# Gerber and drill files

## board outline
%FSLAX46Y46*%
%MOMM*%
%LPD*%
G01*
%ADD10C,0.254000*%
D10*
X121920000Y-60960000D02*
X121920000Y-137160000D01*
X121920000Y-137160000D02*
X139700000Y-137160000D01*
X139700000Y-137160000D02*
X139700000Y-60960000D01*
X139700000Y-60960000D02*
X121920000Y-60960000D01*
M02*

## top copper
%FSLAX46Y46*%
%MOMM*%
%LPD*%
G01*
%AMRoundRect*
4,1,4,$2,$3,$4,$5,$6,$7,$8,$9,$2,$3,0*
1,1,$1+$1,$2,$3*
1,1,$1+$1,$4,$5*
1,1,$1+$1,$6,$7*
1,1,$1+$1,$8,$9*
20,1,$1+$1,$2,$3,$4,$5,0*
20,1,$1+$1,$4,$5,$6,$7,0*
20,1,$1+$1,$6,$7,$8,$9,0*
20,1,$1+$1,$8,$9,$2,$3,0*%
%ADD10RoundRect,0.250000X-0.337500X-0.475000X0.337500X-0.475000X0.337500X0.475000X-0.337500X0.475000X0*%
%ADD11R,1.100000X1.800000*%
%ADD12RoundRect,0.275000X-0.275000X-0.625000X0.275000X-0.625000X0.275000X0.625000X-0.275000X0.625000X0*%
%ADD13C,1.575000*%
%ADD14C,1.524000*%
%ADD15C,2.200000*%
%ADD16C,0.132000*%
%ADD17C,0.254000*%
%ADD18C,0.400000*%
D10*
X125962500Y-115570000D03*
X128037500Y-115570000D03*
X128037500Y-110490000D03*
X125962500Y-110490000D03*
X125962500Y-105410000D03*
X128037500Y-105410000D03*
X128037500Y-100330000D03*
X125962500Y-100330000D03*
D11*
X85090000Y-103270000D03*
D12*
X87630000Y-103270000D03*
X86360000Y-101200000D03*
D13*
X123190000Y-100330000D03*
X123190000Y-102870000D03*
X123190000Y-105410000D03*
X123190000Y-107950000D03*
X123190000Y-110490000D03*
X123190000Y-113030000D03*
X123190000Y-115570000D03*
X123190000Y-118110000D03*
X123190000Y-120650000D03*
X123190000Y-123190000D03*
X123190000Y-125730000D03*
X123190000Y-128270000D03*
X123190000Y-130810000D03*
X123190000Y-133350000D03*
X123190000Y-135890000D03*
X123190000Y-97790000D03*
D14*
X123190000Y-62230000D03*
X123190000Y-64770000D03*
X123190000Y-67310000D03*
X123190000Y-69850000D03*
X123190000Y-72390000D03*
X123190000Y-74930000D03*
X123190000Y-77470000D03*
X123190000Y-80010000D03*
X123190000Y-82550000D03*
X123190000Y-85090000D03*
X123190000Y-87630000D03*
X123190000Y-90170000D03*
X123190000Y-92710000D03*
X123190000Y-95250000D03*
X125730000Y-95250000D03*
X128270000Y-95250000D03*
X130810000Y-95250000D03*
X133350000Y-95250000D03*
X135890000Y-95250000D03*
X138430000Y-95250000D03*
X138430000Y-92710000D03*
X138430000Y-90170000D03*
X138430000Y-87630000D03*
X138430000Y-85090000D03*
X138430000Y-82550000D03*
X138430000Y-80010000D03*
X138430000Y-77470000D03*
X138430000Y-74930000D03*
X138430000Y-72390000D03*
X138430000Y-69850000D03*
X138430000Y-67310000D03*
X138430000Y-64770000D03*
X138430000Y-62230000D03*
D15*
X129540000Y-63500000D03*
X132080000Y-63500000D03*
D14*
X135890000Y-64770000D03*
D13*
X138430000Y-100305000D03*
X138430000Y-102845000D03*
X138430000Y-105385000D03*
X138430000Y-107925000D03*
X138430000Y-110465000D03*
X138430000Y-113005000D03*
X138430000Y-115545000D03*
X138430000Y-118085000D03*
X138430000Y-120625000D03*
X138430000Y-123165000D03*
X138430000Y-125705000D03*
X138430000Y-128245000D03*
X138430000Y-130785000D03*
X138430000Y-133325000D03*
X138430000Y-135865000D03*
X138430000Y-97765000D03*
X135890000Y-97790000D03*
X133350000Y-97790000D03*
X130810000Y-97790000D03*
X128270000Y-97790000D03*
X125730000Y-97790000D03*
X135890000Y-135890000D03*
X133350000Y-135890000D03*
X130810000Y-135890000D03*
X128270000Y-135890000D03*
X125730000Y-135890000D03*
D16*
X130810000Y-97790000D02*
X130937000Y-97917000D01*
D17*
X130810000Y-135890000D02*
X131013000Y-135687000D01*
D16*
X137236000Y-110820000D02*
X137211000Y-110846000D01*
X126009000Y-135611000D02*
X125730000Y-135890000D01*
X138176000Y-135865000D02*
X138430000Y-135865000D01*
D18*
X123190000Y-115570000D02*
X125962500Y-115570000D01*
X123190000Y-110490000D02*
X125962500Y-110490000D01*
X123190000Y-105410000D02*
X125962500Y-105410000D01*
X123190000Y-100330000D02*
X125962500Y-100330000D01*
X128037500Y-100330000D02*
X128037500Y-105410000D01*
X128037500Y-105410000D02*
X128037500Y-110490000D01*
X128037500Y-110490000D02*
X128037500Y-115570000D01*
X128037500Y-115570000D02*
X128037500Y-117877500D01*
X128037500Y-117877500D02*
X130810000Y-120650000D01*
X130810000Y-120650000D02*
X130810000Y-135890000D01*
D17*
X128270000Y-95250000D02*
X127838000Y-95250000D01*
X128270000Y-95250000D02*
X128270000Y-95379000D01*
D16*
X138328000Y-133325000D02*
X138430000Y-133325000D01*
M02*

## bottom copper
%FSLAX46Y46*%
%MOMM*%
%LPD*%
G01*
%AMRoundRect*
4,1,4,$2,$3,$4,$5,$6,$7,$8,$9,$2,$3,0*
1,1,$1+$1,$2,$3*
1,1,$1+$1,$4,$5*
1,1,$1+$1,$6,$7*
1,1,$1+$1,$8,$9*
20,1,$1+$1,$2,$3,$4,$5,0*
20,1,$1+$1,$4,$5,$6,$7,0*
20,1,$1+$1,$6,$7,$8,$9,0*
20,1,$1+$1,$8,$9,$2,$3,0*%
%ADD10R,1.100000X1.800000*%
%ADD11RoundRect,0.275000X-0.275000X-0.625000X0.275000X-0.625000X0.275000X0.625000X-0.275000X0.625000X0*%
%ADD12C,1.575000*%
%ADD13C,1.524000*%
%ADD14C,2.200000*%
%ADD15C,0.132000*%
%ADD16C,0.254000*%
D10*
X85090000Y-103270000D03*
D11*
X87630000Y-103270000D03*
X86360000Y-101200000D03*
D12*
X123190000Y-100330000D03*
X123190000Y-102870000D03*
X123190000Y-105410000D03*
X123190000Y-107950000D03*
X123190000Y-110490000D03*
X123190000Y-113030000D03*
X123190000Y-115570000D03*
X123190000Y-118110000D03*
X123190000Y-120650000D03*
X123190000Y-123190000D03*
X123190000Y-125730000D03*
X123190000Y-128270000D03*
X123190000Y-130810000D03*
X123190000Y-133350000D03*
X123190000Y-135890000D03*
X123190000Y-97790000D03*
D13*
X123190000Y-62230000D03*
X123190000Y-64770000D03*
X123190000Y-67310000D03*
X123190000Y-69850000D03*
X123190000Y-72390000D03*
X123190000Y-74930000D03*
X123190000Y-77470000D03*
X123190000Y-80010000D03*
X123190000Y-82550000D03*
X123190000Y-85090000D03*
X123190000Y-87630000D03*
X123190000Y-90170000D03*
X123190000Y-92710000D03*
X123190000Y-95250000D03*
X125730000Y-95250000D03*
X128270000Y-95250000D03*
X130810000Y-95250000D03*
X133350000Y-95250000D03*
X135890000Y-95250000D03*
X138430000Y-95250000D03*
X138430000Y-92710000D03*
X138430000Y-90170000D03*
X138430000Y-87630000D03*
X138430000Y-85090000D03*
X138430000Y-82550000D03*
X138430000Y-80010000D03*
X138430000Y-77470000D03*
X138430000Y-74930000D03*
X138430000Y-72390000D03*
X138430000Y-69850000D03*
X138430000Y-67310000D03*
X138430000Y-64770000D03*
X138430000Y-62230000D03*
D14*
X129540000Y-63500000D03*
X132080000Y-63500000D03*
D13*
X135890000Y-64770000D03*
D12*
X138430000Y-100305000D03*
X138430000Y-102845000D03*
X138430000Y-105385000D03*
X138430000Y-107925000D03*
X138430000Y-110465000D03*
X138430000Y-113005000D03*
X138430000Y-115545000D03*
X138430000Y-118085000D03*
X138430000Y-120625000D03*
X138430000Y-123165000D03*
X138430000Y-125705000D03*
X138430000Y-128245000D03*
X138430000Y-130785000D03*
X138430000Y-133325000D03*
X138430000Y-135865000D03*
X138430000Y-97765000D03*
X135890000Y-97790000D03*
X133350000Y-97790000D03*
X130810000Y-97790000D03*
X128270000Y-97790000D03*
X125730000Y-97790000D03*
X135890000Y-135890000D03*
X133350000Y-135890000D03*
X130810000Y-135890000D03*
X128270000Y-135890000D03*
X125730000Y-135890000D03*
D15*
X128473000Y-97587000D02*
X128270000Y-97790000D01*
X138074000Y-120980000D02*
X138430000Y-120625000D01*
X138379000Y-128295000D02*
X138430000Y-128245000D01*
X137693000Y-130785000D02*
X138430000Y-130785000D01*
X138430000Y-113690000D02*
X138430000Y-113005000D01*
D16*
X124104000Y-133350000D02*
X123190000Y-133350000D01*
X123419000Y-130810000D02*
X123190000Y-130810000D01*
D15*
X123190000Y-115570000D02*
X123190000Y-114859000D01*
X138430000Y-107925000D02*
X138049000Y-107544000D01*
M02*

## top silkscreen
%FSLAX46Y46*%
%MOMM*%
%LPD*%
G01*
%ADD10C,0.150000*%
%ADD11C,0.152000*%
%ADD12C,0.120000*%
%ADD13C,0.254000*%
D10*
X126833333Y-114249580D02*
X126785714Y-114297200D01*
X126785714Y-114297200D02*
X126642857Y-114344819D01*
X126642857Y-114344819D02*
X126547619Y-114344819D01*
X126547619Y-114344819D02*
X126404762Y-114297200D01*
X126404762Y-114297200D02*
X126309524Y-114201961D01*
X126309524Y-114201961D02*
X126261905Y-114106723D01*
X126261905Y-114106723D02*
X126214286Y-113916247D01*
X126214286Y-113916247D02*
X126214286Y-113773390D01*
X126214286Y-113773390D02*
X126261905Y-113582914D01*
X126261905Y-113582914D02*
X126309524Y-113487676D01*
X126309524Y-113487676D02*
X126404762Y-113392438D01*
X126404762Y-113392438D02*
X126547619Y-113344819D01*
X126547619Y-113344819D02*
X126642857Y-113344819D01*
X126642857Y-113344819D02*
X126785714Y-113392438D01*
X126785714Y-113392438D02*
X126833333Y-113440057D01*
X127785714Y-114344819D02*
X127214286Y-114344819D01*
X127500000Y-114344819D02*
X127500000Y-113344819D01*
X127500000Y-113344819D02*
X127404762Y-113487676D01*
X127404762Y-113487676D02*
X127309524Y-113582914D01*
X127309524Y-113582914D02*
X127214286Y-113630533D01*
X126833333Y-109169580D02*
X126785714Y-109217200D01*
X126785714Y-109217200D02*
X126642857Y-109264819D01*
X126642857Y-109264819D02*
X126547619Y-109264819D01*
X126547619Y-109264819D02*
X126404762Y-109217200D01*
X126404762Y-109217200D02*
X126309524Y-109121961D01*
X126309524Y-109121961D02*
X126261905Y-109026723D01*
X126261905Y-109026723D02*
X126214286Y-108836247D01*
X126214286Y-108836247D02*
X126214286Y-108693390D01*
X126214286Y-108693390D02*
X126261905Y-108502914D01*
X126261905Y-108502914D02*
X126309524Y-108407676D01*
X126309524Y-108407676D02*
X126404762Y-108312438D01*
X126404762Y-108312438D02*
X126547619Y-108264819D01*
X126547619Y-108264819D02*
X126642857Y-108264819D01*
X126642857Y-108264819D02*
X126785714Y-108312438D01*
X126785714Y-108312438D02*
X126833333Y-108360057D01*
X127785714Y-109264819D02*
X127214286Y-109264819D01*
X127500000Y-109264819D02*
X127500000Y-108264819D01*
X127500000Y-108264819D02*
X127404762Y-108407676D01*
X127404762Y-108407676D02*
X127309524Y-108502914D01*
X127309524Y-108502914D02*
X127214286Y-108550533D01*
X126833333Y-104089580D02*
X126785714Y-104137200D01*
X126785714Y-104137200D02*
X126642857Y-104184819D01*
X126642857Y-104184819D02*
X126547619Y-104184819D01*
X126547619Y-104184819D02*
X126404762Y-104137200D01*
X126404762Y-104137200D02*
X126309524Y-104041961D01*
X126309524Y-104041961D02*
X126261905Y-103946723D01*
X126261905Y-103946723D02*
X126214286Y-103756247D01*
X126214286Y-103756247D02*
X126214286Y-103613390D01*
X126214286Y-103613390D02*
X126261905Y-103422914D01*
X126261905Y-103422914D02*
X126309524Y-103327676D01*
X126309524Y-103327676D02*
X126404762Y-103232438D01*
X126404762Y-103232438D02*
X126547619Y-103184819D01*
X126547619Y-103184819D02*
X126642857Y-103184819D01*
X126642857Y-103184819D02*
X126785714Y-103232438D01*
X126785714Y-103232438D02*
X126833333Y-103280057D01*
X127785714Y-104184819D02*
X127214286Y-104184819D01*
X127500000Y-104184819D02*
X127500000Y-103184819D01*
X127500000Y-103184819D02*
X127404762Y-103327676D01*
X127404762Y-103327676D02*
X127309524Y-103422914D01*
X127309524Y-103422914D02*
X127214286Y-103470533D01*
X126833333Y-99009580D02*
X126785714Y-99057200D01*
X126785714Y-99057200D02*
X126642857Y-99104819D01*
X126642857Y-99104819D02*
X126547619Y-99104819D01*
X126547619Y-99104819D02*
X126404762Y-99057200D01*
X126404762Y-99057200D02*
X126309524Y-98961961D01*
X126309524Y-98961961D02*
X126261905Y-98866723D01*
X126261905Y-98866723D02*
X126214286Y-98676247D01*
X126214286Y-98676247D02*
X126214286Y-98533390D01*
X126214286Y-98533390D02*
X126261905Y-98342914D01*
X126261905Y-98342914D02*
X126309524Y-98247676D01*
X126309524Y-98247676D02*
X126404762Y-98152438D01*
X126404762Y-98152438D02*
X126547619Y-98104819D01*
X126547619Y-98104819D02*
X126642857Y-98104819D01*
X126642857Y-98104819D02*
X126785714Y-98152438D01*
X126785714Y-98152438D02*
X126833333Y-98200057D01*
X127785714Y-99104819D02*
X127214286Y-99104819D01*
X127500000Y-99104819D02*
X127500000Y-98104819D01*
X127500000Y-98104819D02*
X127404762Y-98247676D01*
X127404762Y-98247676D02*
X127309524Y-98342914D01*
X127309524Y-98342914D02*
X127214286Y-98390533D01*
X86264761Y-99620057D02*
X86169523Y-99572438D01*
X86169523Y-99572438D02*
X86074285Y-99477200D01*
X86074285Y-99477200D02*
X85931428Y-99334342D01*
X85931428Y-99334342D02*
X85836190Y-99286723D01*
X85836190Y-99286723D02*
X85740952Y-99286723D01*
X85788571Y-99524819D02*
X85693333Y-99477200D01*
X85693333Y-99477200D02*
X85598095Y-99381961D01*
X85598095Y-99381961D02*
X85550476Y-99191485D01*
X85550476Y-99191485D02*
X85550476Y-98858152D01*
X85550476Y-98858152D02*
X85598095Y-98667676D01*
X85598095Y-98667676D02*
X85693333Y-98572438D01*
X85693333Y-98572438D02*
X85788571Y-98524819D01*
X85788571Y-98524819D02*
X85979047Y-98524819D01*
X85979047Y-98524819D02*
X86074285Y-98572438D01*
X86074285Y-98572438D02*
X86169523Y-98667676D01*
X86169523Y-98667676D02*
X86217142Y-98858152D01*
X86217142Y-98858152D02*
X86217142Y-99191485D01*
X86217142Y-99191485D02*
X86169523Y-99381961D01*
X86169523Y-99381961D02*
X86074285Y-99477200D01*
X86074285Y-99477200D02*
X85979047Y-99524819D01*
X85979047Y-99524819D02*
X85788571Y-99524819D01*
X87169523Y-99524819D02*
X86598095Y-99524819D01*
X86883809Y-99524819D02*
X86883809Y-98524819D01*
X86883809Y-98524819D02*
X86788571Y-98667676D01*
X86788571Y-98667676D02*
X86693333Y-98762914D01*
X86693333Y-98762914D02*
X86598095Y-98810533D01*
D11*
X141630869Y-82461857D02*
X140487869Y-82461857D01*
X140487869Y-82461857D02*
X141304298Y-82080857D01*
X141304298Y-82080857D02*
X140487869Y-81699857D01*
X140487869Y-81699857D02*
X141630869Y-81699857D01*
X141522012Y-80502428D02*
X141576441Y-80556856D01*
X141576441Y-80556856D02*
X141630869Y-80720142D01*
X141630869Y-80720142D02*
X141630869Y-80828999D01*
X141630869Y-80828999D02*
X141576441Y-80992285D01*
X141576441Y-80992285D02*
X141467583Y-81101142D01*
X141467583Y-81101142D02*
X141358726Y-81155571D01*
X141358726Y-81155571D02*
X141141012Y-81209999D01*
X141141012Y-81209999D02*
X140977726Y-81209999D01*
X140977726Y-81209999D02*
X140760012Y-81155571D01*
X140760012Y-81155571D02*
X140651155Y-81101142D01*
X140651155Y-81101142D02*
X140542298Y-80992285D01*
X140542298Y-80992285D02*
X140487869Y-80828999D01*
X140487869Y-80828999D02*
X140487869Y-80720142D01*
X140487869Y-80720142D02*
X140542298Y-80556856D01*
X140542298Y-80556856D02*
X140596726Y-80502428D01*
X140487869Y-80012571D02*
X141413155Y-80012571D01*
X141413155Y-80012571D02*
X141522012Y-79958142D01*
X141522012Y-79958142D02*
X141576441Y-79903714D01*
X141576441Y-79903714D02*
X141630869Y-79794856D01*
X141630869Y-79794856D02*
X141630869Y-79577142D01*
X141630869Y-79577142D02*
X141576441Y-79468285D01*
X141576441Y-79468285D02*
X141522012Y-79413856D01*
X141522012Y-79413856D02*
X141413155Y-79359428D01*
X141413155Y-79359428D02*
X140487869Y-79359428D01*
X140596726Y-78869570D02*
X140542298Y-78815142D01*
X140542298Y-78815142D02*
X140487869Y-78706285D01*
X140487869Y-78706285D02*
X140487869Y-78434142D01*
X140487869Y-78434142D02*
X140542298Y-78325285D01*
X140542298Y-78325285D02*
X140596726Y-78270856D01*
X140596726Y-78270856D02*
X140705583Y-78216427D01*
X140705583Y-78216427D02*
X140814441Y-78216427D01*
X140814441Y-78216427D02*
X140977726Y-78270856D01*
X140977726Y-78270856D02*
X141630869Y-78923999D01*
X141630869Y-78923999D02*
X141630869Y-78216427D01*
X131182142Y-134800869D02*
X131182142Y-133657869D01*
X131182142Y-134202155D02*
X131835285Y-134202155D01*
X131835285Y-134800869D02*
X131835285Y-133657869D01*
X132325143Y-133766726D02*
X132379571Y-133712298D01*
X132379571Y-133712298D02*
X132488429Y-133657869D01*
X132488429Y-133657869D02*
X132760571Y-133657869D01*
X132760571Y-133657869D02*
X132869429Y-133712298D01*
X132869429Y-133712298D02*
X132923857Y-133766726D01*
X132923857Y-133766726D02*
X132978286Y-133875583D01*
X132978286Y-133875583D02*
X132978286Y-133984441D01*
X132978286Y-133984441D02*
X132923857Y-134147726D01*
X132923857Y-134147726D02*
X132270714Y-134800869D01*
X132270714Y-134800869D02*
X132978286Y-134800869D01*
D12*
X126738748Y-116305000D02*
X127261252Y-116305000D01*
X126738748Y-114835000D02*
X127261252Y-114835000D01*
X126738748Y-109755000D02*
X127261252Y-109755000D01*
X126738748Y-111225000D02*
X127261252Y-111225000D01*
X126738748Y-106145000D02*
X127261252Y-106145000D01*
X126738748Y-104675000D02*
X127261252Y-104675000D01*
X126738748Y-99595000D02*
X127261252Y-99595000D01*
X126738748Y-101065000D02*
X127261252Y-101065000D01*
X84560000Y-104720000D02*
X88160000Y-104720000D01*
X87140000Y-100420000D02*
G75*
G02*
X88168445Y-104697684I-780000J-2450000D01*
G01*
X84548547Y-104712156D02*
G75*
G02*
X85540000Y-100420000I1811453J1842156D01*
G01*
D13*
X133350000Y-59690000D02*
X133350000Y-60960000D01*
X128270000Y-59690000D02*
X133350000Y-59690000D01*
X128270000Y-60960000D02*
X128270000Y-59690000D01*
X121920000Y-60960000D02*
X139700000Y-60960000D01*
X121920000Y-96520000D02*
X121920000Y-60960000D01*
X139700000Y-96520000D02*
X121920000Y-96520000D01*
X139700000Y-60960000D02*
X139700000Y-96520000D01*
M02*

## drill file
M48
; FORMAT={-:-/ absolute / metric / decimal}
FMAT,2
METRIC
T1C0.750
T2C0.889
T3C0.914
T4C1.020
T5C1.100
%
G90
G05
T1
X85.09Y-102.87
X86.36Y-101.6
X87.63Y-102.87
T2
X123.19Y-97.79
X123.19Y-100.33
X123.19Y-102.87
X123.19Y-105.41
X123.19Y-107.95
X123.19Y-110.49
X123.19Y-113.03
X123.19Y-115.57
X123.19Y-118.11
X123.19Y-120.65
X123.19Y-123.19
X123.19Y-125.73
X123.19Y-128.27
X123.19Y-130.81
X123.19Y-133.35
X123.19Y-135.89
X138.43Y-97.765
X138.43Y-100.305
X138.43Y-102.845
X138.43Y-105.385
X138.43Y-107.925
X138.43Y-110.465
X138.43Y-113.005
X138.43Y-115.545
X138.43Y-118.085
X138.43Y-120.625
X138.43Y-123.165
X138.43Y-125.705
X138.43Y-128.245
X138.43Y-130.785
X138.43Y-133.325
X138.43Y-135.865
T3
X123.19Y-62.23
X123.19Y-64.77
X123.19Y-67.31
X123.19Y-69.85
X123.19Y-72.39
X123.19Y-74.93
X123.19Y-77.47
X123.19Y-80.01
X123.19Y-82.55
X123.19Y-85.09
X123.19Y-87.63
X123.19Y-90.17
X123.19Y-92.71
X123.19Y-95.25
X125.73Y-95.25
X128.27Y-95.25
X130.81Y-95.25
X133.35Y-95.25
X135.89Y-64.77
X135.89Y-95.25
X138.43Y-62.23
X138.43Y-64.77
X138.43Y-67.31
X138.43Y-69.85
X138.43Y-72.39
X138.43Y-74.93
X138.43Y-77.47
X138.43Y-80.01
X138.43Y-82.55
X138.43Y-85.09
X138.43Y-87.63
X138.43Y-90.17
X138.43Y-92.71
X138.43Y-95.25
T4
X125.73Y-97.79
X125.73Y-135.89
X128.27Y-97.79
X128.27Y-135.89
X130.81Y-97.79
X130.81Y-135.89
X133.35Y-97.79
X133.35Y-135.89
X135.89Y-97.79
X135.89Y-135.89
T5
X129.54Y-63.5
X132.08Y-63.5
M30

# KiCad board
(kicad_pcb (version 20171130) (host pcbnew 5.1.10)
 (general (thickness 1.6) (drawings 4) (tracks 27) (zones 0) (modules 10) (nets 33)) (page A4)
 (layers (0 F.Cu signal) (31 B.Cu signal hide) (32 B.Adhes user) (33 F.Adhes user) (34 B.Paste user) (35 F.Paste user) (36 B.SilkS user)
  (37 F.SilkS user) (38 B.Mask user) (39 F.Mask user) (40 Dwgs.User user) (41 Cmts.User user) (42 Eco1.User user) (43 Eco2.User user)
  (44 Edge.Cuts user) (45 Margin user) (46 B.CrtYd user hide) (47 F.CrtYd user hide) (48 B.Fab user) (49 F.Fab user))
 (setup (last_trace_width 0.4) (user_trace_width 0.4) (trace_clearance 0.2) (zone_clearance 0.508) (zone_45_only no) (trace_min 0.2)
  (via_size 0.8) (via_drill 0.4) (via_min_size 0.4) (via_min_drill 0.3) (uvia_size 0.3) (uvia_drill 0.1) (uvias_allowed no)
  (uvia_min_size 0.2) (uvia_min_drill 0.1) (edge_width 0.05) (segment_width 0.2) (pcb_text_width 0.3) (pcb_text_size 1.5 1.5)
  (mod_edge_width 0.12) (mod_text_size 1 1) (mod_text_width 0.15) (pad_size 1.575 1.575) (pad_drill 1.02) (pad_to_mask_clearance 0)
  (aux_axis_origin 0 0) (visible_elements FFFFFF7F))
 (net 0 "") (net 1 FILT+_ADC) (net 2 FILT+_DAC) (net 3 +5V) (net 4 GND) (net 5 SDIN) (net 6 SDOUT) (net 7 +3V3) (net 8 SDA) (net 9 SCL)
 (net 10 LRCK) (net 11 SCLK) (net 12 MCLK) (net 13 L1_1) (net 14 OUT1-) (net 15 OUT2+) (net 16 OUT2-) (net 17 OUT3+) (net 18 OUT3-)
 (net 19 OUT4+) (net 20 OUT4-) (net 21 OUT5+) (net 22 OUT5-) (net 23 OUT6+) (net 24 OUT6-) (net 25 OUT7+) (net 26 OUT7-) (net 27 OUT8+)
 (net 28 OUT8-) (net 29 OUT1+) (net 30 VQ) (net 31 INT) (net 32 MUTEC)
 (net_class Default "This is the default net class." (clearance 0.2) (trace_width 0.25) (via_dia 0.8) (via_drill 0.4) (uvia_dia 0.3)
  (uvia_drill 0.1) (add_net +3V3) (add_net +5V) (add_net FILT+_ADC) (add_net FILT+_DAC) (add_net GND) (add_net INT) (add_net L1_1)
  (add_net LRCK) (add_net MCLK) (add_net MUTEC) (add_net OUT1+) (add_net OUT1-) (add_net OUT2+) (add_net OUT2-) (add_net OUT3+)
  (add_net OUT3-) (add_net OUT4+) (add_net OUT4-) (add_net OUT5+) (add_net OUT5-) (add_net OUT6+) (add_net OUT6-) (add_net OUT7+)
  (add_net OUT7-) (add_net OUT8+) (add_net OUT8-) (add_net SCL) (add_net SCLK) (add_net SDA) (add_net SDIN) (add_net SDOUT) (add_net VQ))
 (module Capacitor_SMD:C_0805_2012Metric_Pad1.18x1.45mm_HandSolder (layer F.Cu) (at 127 115.57)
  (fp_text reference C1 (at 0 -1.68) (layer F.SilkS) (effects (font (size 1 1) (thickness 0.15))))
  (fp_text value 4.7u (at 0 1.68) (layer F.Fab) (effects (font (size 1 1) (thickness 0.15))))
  (fp_line (start -0.261252 0.735) (end 0.261252 0.735) (layer F.SilkS) (width 0.12))
  (fp_line (start -0.261252 -0.735) (end 0.261252 -0.735) (layer F.SilkS) (width 0.12))
  (pad 1 smd roundrect (at -1.0375 0) (size 1.175 1.45) (layers F.Cu F.Paste F.Mask) (roundrect_rratio 0.212766))
  (pad 2 smd roundrect (at 1.0375 0) (size 1.175 1.45) (layers F.Cu F.Paste F.Mask) (roundrect_rratio 0.212766)))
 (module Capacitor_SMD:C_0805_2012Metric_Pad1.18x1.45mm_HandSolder (layer F.Cu) (at 127 110.49)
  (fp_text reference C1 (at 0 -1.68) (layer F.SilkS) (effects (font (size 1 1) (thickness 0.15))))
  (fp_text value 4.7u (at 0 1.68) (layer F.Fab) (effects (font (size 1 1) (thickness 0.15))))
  (fp_line (start -0.261252 -0.735) (end 0.261252 -0.735) (layer F.SilkS) (width 0.12))
  (fp_line (start -0.261252 0.735) (end 0.261252 0.735) (layer F.SilkS) (width 0.12))
  (pad 2 smd roundrect (at 1.0375 0) (size 1.175 1.45) (layers F.Cu F.Paste F.Mask) (roundrect_rratio 0.212766))
  (pad 1 smd roundrect (at -1.0375 0) (size 1.175 1.45) (layers F.Cu F.Paste F.Mask) (roundrect_rratio 0.212766)))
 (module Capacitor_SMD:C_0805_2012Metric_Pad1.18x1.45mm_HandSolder (layer F.Cu) (at 127 105.41)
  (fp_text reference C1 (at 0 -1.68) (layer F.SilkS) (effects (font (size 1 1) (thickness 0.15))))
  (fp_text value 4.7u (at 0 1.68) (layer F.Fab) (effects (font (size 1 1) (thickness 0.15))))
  (fp_line (start -0.261252 0.735) (end 0.261252 0.735) (layer F.SilkS) (width 0.12))
  (fp_line (start -0.261252 -0.735) (end 0.261252 -0.735) (layer F.SilkS) (width 0.12))
  (pad 1 smd roundrect (at -1.0375 0) (size 1.175 1.45) (layers F.Cu F.Paste F.Mask) (roundrect_rratio 0.212766))
  (pad 2 smd roundrect (at 1.0375 0) (size 1.175 1.45) (layers F.Cu F.Paste F.Mask) (roundrect_rratio 0.212766)))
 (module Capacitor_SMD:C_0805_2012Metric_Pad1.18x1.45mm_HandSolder (layer F.Cu) (at 127 100.33)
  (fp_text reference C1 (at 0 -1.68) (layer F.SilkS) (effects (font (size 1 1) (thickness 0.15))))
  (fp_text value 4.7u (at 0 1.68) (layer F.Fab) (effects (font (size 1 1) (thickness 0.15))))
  (fp_line (start -0.261252 -0.735) (end 0.261252 -0.735) (layer F.SilkS) (width 0.12))
  (fp_line (start -0.261252 0.735) (end 0.261252 0.735) (layer F.SilkS) (width 0.12))
  (pad 2 smd roundrect (at 1.0375 0) (size 1.175 1.45) (layers F.Cu F.Paste F.Mask) (roundrect_rratio 0.212766))
  (pad 1 smd roundrect (at -1.0375 0) (size 1.175 1.45) (layers F.Cu F.Paste F.Mask) (roundrect_rratio 0.212766)))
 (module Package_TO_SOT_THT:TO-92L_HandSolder (layer F.Cu) (at 85.09 102.87)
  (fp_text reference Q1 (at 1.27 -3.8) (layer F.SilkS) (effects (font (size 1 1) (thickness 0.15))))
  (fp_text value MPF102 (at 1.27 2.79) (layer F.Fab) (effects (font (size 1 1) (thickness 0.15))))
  (fp_line (start -0.53 1.85) (end 3.07 1.85) (layer F.SilkS) (width 0.12))
  (fp_arc (start 1.27 0) (end 2.05 -2.45) (angle 117.6433766) (layer F.SilkS) (width 0.12))
  (fp_arc (start 1.27 0) (end 0.45 -2.45) (angle -116.9763941) (layer F.SilkS) (width 0.12))
  (pad D thru_hole rect (at 0 0) (size 1.1 1.8) (drill 0.75 (offset 0 0.4)) (layers *.Cu *.Mask))
  (pad G thru_hole roundrect (at 2.54 0) (size 1.1 1.8) (drill 0.75 (offset 0 0.4)) (layers *.Cu *.Mask) (roundrect_rratio 0.25))
  (pad S thru_hole roundrect (at 1.27 -1.27) (size 1.1 1.8) (drill 0.75 (offset 0 -0.4)) (layers *.Cu *.Mask) (roundrect_rratio 0.25)))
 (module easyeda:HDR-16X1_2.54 (layer F.Cu) (at 123.19 116.84)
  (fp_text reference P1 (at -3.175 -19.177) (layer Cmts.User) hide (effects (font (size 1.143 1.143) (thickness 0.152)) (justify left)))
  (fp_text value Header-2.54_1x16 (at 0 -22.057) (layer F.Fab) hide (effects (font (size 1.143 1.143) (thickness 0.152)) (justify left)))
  (pad I1- thru_hole circle (at 0 -16.51 270) (size 1.575 1.575) (drill 0.889) (layers *.Cu *.Paste *.Mask))
  (pad I2+ thru_hole circle (at 0 -13.97 270) (size 1.575 1.575) (drill 0.889) (layers *.Cu *.Paste *.Mask))
  (pad I2- thru_hole circle (at 0 -11.43 270) (size 1.575 1.575) (drill 0.889) (layers *.Cu *.Paste *.Mask))
  (pad I3+ thru_hole circle (at 0 -8.89 270) (size 1.575 1.575) (drill 0.889) (layers *.Cu *.Paste *.Mask))
  (pad I3- thru_hole circle (at 0 -6.35 270) (size 1.575 1.575) (drill 0.889) (layers *.Cu *.Paste *.Mask))
  (pad I4+ thru_hole circle (at 0 -3.81 270) (size 1.575 1.575) (drill 0.889) (layers *.Cu *.Paste *.Mask))
  (pad I4- thru_hole circle (at 0 -1.27 270) (size 1.575 1.575) (drill 0.889) (layers *.Cu *.Paste *.Mask))
  (pad I5+ thru_hole circle (at 0 1.27 270) (size 1.575 1.575) (drill 0.889) (layers *.Cu *.Paste *.Mask))
  (pad I5- thru_hole circle (at 0 3.81 270) (size 1.575 1.575) (drill 0.889) (layers *.Cu *.Paste *.Mask))
  (pad I6+ thru_hole circle (at 0 6.35 270) (size 1.575 1.575) (drill 0.889) (layers *.Cu *.Paste *.Mask))
  (pad I6- thru_hole circle (at 0 8.89 270) (size 1.575 1.575) (drill 0.889) (layers *.Cu *.Paste *.Mask))
  (pad 13 thru_hole circle (at 0 11.43 270) (size 1.575 1.575) (drill 0.889) (layers *.Cu *.Paste *.Mask) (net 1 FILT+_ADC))
  (pad 14 thru_hole circle (at 0 13.97 270) (size 1.575 1.575) (drill 0.889) (layers *.Cu *.Paste *.Mask) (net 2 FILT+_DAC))
  (pad 15 thru_hole circle (at 0 16.51 270) (size 1.575 1.575) (drill 0.889) (layers *.Cu *.Paste *.Mask) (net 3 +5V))
  (pad 16 thru_hole circle (at 0 19.05 270) (size 1.575 1.575) (drill 0.889) (layers *.Cu *.Paste *.Mask) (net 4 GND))
  (pad I1+ thru_hole circle (at 0 -19.05 270) (size 1.575 1.575) (drill 0.889) (layers *.Cu *.Paste *.Mask)))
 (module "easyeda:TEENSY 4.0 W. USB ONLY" (layer F.Cu) (at 123.19 62.23 270)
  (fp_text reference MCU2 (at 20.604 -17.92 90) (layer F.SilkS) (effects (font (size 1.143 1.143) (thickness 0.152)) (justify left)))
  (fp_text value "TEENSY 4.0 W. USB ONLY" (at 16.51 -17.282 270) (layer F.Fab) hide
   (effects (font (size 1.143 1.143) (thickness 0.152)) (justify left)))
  (fp_line (start -2.54 -10.16) (end -1.27 -10.16) (layer F.SilkS) (width 0.254))
  (fp_line (start -2.54 -5.08) (end -2.54 -10.16) (layer F.SilkS) (width 0.254))
  (fp_line (start -1.27 -5.08) (end -2.54 -5.08) (layer F.SilkS) (width 0.254))
  (fp_line (start -1.27 1.27) (end -1.27 -16.51) (layer F.SilkS) (width 0.254))
  (fp_line (start 34.29 1.27) (end -1.27 1.27) (layer F.SilkS) (width 0.254))
  (fp_line (start 34.29 -16.51) (end 34.29 1.27) (layer F.SilkS) (width 0.254))
  (fp_line (start -1.27 -16.51) (end 34.29 -16.51) (layer F.SilkS) (width 0.254))
  (pad GND0 thru_hole circle (at 0 0 270) (size 1.524 1.524) (drill 0.914) (layers *.Cu *.Paste *.Mask) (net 4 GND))
  (pad 0 thru_hole circle (at 2.54 0 270) (size 1.524 1.524) (drill 0.914) (layers *.Cu *.Paste *.Mask))
  (pad 1 thru_hole circle (at 5.08 0 270) (size 1.524 1.524) (drill 0.914) (layers *.Cu *.Paste *.Mask))
  (pad 2 thru_hole circle (at 7.62 0 270) (size 1.524 1.524) (drill 0.914) (layers *.Cu *.Paste *.Mask))
  (pad 3 thru_hole circle (at 10.16 0 270) (size 1.524 1.524) (drill 0.914) (layers *.Cu *.Paste *.Mask))
  (pad 4 thru_hole circle (at 12.7 0 270) (size 1.524 1.524) (drill 0.914) (layers *.Cu *.Paste *.Mask))
  (pad 5 thru_hole circle (at 15.24 0 270) (size 1.524 1.524) (drill 0.914) (layers *.Cu *.Paste *.Mask))
  (pad 6 thru_hole circle (at 17.78 0 270) (size 1.524 1.524) (drill 0.914) (layers *.Cu *.Paste *.Mask))
  (pad 7 thru_hole circle (at 20.32 0 270) (size 1.524 1.524) (drill 0.914) (layers *.Cu *.Paste *.Mask) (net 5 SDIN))
  (pad 8 thru_hole circle (at 22.86 0 270) (size 1.524 1.524) (drill 0.914) (layers *.Cu *.Paste *.Mask) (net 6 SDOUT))
  (pad 9 thru_hole circle (at 25.4 0 270) (size 1.524 1.524) (drill 0.914) (layers *.Cu *.Paste *.Mask))
  (pad 10 thru_hole circle (at 27.94 0 270) (size 1.524 1.524) (drill 0.914) (layers *.Cu *.Paste *.Mask))
  (pad 11 thru_hole circle (at 30.48 0 270) (size 1.524 1.524) (drill 0.914) (layers *.Cu *.Paste *.Mask))
  (pad 12 thru_hole circle (at 33.02 0 270) (size 1.524 1.524) (drill 0.914) (layers *.Cu *.Paste *.Mask))
  (pad VBAT thru_hole circle (at 33.02 -2.54 270) (size 1.524 1.524) (drill 0.914) (layers *.Cu *.Paste *.Mask))
  (pad 3 thru_hole circle (at 33.02 -5.08 270) (size 1.524 1.524) (drill 0.914) (layers *.Cu *.Paste *.Mask) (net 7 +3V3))
  (pad GND2 thru_hole circle (at 33.02 -7.62 270) (size 1.524 1.524) (drill 0.914) (layers *.Cu *.Paste *.Mask) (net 4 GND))
  (pad PRGM thru_hole circle (at 33.02 -10.16 270) (size 1.524 1.524) (drill 0.914) (layers *.Cu *.Paste *.Mask))
  (pad ONOFF thru_hole circle (at 33.02 -12.7 270) (size 1.524 1.524) (drill 0.914) (layers *.Cu *.Paste *.Mask))
  (pad 13 thru_hole circle (at 33.02 -15.24 270) (size 1.524 1.524) (drill 0.914) (layers *.Cu *.Paste *.Mask))
  (pad 14 thru_hole circle (at 30.48 -15.24 270) (size 1.524 1.524) (drill 0.914) (layers *.Cu *.Paste *.Mask))
  (pad 15 thru_hole circle (at 27.94 -15.24 270) (size 1.524 1.524) (drill 0.914) (layers *.Cu *.Paste *.Mask))
  (pad 16 thru_hole circle (at 25.4 -15.24 270) (size 1.524 1.524) (drill 0.914) (layers *.Cu *.Paste *.Mask))
  (pad 17 thru_hole circle (at 22.86 -15.24 270) (size 1.524 1.524) (drill 0.914) (layers *.Cu *.Paste *.Mask))
  (pad 18 thru_hole circle (at 20.32 -15.24 270) (size 1.524 1.524) (drill 0.914) (layers *.Cu *.Paste *.Mask) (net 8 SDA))
  (pad 19 thru_hole circle (at 17.78 -15.24 270) (size 1.524 1.524) (drill 0.914) (layers *.Cu *.Paste *.Mask) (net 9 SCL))
  (pad 20 thru_hole circle (at 15.24 -15.24 270) (size 1.524 1.524) (drill 0.914) (layers *.Cu *.Paste *.Mask) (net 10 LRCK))
  (pad 21 thru_hole circle (at 12.7 -15.24 270) (size 1.524 1.524) (drill 0.914) (layers *.Cu *.Paste *.Mask) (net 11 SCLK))
  (pad 22 thru_hole circle (at 10.16 -15.24 270) (size 1.524 1.524) (drill 0.914) (layers *.Cu *.Paste *.Mask))
  (pad 23 thru_hole circle (at 7.62 -15.24 270) (size 1.524 1.524) (drill 0.914) (layers *.Cu *.Paste *.Mask) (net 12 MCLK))
  (pad 3 thru_hole circle (at 5.08 -15.24 270) (size 1.524 1.524) (drill 0.914) (layers *.Cu *.Paste *.Mask) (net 7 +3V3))
  (pad GND1 thru_hole circle (at 2.54 -15.24 270) (size 1.524 1.524) (drill 0.914) (layers *.Cu *.Paste *.Mask) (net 4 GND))
  (pad VIN thru_hole circle (at 0 -15.24 270) (size 1.524 1.524) (drill 0.914) (layers *.Cu *.Paste *.Mask) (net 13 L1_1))
  (pad D+ thru_hole circle (at 1.27 -6.35 270) (size 2.2 2.2) (drill 1.1) (layers *.Cu *.Paste *.Mask))
  (pad D- thru_hole circle (at 1.27 -8.89 270) (size 2.2 2.2) (drill 1.1) (layers *.Cu *.Paste *.Mask))
  (pad VUSB thru_hole circle (at 2.54 -12.7 270) (size 1.524 1.524) (drill 0.914) (layers *.Cu *.Paste *.Mask)))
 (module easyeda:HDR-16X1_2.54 (layer F.Cu) (at 138.43 116.815)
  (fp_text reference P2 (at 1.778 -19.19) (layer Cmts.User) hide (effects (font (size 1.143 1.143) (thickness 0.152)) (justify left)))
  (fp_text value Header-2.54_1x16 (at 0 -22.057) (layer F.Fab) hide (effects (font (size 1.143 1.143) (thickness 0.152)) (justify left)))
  (pad 2 thru_hole circle (at 0 -16.51 270) (size 1.575 1.575) (drill 0.889) (layers *.Cu *.Paste *.Mask) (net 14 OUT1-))
  (pad 3 thru_hole circle (at 0 -13.97 270) (size 1.575 1.575) (drill 0.889) (layers *.Cu *.Paste *.Mask) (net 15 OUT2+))
  (pad 4 thru_hole circle (at 0 -11.43 270) (size 1.575 1.575) (drill 0.889) (layers *.Cu *.Paste *.Mask) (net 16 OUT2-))
  (pad 5 thru_hole circle (at 0 -8.89 270) (size 1.575 1.575) (drill 0.889) (layers *.Cu *.Paste *.Mask) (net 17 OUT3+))
  (pad 6 thru_hole circle (at 0 -6.35 270) (size 1.575 1.575) (drill 0.889) (layers *.Cu *.Paste *.Mask) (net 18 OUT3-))
  (pad 7 thru_hole circle (at 0 -3.81 270) (size 1.575 1.575) (drill 0.889) (layers *.Cu *.Paste *.Mask) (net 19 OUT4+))
  (pad 8 thru_hole circle (at 0 -1.27 270) (size 1.575 1.575) (drill 0.889) (layers *.Cu *.Paste *.Mask) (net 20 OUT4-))
  (pad 9 thru_hole circle (at 0 1.27 270) (size 1.575 1.575) (drill 0.889) (layers *.Cu *.Paste *.Mask) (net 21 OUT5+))
  (pad 10 thru_hole circle (at 0 3.81 270) (size 1.575 1.575) (drill 0.889) (layers *.Cu *.Paste *.Mask) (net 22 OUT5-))
  (pad 11 thru_hole circle (at 0 6.35 270) (size 1.575 1.575) (drill 0.889) (layers *.Cu *.Paste *.Mask) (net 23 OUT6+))
  (pad 12 thru_hole circle (at 0 8.89 270) (size 1.575 1.575) (drill 0.889) (layers *.Cu *.Paste *.Mask) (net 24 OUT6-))
  (pad 13 thru_hole circle (at 0 11.43 270) (size 1.575 1.575) (drill 0.889) (layers *.Cu *.Paste *.Mask) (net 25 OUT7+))
  (pad 14 thru_hole circle (at 0 13.97 270) (size 1.575 1.575) (drill 0.889) (layers *.Cu *.Paste *.Mask) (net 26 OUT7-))
  (pad 15 thru_hole circle (at 0 16.51 270) (size 1.575 1.575) (drill 0.889) (layers *.Cu *.Paste *.Mask) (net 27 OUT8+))
  (pad 16 thru_hole circle (at 0 19.05 270) (size 1.575 1.575) (drill 0.889) (layers *.Cu *.Paste *.Mask) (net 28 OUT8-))
  (pad 1 thru_hole circle (at 0 -19.05 270) (size 1.575 1.575) (drill 0.889) (layers *.Cu *.Paste *.Mask) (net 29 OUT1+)))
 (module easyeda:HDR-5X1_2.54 (layer F.Cu) (at 130.81 97.79)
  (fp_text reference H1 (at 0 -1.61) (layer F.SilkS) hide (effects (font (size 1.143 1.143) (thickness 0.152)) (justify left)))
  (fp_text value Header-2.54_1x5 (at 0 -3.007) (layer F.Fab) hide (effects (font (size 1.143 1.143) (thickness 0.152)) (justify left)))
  (pad 5 thru_hole circle (at 5.08 0) (size 1.575 1.575) (drill 1.02) (layers *.Cu *.Paste *.Mask) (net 6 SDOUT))
  (pad 4 thru_hole circle (at 2.54 0) (size 1.575 1.575) (drill 1.02) (layers *.Cu *.Paste *.Mask) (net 5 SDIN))
  (pad 3 thru_hole circle (at 0 0) (size 1.575 1.575) (drill 1.02) (layers *.Cu *.Paste *.Mask) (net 10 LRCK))
  (pad 2 thru_hole circle (at -2.54 0) (size 1.575 1.575) (drill 1.02) (layers *.Cu *.Paste *.Mask) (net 11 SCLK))
  (pad 1 thru_hole circle (at -5.08 0) (size 1.575 1.575) (drill 1.02) (layers *.Cu *.Paste *.Mask) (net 12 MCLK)))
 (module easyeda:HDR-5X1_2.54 (layer F.Cu) (at 130.81 135.89)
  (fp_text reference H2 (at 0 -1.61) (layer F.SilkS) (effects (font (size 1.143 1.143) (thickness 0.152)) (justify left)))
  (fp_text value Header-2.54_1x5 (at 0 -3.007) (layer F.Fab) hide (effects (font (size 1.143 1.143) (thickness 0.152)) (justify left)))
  (pad 5 thru_hole circle (at 5.08 0) (size 1.575 1.575) (drill 1.02) (layers *.Cu *.Paste *.Mask) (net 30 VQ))
  (pad 4 thru_hole circle (at 2.54 0) (size 1.575 1.575) (drill 1.02) (layers *.Cu *.Paste *.Mask) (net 3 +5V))
  (pad GND thru_hole circle (at 0 0) (size 1.575 1.575) (drill 1.02) (layers *.Cu *.Paste *.Mask))
  (pad 2 thru_hole circle (at -2.54 0) (size 1.575 1.575) (drill 1.02) (layers *.Cu *.Paste *.Mask) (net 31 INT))
  (pad 1 thru_hole circle (at -5.08 0) (size 1.575 1.575) (drill 1.02) (layers *.Cu *.Paste *.Mask) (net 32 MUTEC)))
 (gr_line (start 121.92 60.96) (end 121.92 137.16) (layer Edge.Cuts) (width 0.254))
 (gr_line (start 121.92 137.16) (end 139.7 137.16) (layer Edge.Cuts) (width 0.254))
 (gr_line (start 139.7 137.16) (end 139.7 60.96) (layer Edge.Cuts) (width 0.254))
 (gr_line (start 139.7 60.96) (end 121.92 60.96) (layer Edge.Cuts) (width 0.254))
 (segment (start 130.81 97.79) (end 130.937 97.917) (width 0.132) (layer F.Cu) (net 10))
 (segment (start 128.473 97.587) (end 128.27 97.79) (width 0.132) (layer B.Cu) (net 11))
 (segment (start 130.81 135.89) (end 131.013 135.687) (width 0.254) (layer F.Cu) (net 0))
 (segment (start 137.236 110.82) (end 137.211 110.846) (width 0.132) (layer F.Cu) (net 4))
 (segment (start 126.009 135.611) (end 125.73 135.89) (width 0.132) (layer F.Cu) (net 32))
 (segment (start 138.074 120.98) (end 138.43 120.625) (width 0.132) (layer B.Cu) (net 22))
 (segment (start 138.379 128.295) (end 138.43 128.245) (width 0.132) (layer B.Cu) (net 25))
 (segment (start 138.176 135.865) (end 138.43 135.865) (width 0.132) (layer F.Cu) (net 28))
 (segment (start 137.693 130.785) (end 138.43 130.785) (width 0.132) (layer B.Cu) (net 26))
 (segment (start 138.43 113.69) (end 138.43 113.005) (width 0.132) (layer B.Cu) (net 19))
 (segment (start 124.104 133.35) (end 123.19 133.35) (width 0.254) (layer B.Cu) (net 3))
 (segment (start 123.419 130.81) (end 123.19 130.81) (width 0.254) (layer B.Cu) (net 2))
 (segment (start 123.19 115.57) (end 123.19 114.859) (width 0.132) (layer B.Cu) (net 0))
 (segment (start 123.19 115.57) (end 125.9625 115.57) (width 0.4) (layer F.Cu) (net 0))
 (segment (start 123.19 110.49) (end 125.9625 110.49) (width 0.4) (layer F.Cu) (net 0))
 (segment (start 123.19 105.41) (end 125.9625 105.41) (width 0.4) (layer F.Cu) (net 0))
 (segment (start 123.19 100.33) (end 125.9625 100.33) (width 0.4) (layer F.Cu) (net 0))
 (segment (start 128.0375 100.33) (end 128.0375 105.41) (width 0.4) (layer F.Cu) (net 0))
 (segment (start 128.0375 105.41) (end 128.0375 110.49) (width 0.4) (layer F.Cu) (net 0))
 (segment (start 128.0375 110.49) (end 128.0375 115.57) (width 0.4) (layer F.Cu) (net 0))
 (segment (start 128.0375 115.57) (end 128.0375 117.8775) (width 0.4) (layer F.Cu) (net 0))
 (segment (start 128.0375 117.8775) (end 130.81 120.65) (width 0.4) (layer F.Cu) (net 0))
 (segment (start 130.81 120.65) (end 130.81 135.89) (width 0.4) (layer F.Cu) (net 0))
 (segment (start 138.43 107.925) (end 138.049 107.544) (width 0.132) (layer B.Cu) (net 17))
 (segment (start 128.27 95.25) (end 127.838 95.25) (width 0.254) (layer F.Cu) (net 7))
 (segment (start 128.27 95.25) (end 128.27 95.379) (width 0.254) (layer F.Cu) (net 7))
 (segment (start 138.328 133.325) (end 138.43 133.325) (width 0.132) (layer F.Cu) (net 27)))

